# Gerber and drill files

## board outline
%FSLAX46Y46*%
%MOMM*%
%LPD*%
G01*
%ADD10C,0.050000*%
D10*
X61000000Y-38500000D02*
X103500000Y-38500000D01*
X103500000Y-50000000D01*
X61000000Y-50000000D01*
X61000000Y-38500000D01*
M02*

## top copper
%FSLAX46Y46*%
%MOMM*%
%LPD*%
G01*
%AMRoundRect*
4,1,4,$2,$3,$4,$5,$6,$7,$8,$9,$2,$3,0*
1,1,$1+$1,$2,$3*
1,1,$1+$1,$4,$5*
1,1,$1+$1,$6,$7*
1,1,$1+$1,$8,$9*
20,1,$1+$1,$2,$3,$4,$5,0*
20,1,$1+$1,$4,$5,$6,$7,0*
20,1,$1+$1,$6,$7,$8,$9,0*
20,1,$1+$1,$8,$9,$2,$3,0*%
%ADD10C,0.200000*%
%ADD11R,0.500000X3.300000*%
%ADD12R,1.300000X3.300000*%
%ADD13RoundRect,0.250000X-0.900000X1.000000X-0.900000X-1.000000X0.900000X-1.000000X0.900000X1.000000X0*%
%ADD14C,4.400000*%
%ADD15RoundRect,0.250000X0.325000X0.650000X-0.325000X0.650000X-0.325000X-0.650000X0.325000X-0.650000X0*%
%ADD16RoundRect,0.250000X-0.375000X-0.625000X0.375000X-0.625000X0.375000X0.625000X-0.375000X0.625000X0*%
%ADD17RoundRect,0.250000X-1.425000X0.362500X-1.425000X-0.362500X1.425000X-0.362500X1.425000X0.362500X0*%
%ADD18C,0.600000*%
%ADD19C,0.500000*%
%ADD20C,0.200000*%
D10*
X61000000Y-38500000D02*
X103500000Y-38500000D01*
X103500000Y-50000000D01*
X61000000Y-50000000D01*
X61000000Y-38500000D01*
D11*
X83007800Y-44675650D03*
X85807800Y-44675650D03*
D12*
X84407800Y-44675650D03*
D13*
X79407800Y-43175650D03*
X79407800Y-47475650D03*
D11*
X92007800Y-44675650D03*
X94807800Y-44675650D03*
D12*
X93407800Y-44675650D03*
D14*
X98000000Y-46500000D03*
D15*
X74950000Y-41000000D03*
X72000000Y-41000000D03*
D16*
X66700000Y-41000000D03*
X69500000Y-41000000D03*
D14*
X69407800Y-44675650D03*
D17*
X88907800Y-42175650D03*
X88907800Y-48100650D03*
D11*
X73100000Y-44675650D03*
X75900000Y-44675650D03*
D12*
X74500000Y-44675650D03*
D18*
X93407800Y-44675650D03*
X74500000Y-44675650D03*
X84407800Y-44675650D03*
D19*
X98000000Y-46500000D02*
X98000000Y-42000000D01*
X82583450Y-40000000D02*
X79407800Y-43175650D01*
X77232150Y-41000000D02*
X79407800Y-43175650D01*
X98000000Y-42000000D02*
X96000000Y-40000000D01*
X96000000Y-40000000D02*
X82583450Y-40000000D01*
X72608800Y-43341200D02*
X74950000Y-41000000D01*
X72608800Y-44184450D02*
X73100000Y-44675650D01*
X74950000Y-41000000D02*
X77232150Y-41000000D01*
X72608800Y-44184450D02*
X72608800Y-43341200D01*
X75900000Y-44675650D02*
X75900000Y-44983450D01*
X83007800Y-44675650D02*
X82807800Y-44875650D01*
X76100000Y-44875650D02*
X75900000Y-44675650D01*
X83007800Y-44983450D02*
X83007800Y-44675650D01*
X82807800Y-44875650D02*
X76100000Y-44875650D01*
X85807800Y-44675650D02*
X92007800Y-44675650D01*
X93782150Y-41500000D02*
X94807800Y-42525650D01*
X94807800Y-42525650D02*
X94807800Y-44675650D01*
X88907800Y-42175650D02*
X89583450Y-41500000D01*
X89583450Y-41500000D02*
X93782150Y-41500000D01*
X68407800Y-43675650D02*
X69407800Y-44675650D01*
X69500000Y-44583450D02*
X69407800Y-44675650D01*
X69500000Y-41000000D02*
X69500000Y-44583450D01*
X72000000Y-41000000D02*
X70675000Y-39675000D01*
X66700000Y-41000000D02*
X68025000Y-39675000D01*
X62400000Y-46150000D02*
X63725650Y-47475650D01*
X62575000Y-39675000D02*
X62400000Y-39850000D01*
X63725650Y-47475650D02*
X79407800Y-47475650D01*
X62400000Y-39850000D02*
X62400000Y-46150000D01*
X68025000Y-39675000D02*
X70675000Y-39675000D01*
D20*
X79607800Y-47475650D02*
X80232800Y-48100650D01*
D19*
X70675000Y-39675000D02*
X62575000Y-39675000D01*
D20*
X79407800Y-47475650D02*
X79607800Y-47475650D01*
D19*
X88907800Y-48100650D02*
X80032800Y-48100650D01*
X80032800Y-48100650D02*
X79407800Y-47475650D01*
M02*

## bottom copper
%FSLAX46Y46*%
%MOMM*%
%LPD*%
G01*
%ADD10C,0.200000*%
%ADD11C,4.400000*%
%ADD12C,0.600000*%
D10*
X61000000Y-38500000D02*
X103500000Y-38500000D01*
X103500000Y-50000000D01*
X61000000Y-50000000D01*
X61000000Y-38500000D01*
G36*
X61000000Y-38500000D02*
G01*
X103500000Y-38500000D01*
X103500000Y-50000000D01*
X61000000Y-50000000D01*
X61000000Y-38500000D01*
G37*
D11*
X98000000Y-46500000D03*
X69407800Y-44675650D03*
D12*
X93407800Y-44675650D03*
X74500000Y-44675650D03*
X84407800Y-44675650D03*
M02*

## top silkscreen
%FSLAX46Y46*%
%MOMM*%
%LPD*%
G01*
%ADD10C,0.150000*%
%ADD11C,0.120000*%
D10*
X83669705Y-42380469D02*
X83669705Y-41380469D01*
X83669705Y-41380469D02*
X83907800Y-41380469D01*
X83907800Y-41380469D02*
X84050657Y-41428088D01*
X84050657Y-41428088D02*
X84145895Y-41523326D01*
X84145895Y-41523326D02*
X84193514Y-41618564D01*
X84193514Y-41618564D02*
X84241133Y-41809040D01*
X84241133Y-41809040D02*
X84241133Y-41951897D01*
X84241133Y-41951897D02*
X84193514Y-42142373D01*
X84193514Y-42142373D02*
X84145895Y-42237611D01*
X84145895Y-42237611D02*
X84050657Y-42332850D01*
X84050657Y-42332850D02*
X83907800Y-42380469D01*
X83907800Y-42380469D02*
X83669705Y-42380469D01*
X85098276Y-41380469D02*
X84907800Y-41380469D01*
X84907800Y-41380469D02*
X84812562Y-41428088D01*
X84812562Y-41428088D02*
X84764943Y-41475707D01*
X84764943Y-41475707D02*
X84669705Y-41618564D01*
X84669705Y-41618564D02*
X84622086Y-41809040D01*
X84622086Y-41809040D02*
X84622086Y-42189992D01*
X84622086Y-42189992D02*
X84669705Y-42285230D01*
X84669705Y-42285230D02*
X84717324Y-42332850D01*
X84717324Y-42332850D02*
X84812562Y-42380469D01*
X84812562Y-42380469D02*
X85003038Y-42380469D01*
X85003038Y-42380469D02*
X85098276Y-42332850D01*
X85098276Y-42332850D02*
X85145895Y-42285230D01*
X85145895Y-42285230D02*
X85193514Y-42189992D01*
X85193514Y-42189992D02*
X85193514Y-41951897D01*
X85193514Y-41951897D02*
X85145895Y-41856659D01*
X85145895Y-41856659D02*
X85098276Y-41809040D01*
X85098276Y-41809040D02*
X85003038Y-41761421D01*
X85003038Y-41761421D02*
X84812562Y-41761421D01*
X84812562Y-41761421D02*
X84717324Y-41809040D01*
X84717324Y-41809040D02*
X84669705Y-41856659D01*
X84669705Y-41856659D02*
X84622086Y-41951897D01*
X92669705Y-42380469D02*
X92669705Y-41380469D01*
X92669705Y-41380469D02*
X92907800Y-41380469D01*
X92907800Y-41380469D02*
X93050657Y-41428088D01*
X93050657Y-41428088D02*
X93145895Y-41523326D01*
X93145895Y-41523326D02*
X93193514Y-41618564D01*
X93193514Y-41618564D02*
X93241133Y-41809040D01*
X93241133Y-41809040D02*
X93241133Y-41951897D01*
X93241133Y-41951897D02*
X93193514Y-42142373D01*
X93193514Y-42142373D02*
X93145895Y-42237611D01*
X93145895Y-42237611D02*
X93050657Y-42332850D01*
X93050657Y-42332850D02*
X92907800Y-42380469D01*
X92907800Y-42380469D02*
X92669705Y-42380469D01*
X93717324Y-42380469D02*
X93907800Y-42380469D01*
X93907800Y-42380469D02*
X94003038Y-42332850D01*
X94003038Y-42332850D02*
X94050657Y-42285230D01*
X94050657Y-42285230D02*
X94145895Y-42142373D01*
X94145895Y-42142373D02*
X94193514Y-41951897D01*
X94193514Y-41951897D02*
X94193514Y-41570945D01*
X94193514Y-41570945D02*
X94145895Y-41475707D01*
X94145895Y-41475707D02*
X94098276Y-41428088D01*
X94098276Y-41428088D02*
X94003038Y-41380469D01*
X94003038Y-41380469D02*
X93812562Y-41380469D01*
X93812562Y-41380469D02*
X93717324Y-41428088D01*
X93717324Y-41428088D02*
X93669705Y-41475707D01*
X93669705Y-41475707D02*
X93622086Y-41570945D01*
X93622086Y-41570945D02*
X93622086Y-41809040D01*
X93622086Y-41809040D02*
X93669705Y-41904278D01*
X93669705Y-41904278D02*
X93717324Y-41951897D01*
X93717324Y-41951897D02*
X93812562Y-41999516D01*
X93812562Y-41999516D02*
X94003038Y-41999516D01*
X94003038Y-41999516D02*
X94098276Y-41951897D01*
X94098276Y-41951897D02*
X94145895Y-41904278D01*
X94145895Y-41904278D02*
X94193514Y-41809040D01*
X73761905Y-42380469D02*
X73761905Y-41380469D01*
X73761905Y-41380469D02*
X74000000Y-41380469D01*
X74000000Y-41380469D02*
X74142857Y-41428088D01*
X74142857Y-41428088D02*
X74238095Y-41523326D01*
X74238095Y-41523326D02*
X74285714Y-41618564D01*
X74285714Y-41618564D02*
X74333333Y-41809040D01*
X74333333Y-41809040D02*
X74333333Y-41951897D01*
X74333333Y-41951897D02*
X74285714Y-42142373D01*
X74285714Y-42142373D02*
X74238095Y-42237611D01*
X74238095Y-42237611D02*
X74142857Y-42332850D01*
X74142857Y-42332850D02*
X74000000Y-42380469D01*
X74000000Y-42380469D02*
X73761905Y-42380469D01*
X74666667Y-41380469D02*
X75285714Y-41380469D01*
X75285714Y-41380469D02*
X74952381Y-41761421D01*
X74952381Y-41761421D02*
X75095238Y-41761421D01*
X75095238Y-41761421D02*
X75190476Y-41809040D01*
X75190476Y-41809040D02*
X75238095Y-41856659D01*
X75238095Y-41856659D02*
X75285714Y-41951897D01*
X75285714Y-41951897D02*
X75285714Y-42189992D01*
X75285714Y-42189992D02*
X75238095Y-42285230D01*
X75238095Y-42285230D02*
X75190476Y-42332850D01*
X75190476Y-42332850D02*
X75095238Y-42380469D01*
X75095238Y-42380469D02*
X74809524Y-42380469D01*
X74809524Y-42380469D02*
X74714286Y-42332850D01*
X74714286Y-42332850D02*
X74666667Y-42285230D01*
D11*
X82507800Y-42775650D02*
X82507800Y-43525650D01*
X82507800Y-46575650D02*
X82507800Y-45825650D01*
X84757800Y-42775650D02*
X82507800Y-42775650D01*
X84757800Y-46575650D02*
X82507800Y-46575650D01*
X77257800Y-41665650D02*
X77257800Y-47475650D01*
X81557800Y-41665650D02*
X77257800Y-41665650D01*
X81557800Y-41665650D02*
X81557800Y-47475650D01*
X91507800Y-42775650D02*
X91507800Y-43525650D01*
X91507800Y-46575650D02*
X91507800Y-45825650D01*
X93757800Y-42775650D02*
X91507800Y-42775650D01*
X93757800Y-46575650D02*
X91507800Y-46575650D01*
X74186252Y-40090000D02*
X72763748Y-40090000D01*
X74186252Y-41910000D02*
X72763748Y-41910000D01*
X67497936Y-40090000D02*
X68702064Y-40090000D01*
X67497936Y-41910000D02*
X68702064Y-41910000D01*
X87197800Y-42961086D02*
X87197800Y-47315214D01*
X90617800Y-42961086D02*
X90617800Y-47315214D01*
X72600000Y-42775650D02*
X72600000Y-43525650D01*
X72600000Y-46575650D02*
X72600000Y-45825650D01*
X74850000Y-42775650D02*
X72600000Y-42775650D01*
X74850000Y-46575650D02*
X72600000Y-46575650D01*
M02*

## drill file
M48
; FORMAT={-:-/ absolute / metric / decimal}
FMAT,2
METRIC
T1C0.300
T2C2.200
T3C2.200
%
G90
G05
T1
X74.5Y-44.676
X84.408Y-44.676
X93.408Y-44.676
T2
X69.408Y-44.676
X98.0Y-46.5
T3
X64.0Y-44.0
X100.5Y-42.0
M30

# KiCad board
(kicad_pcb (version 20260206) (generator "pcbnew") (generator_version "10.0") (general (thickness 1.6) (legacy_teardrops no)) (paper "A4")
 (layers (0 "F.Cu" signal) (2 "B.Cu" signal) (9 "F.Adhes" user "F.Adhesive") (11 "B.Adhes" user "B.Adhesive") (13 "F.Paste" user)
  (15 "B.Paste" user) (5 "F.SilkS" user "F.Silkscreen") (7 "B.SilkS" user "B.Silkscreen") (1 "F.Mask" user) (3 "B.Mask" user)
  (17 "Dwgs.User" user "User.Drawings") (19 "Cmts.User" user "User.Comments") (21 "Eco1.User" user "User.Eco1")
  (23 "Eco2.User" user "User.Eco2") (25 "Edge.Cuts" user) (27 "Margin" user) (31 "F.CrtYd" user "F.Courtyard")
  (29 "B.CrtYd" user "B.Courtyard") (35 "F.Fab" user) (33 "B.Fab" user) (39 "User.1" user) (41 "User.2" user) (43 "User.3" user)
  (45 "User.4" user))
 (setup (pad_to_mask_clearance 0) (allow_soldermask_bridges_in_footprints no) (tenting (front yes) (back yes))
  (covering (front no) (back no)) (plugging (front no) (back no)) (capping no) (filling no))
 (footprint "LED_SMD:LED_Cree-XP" (layer "F.Cu") (at 84.4078 44.67565)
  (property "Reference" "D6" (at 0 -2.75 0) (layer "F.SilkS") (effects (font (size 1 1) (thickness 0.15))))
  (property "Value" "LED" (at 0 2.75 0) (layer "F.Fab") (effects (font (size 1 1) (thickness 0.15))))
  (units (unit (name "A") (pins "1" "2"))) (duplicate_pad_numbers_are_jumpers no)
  (fp_line (start -1.9 -1.9) (end -1.9 -1.15) (stroke (width 0.12) (type solid)) (layer "F.SilkS"))
  (fp_line (start -1.9 1.9) (end -1.9 1.15) (stroke (width 0.12) (type solid)) (layer "F.SilkS"))
  (fp_line (start 0.35 -1.9) (end -1.9 -1.9) (stroke (width 0.12) (type solid)) (layer "F.SilkS"))
  (fp_line (start 0.35 1.9) (end -1.9 1.9) (stroke (width 0.12) (type solid)) (layer "F.SilkS"))
  (pad "" smd rect (at 0 -1) (size 1.01 0.75) (layers "F.Paste"))
  (pad "" smd rect (at 0 0) (size 1.01 0.75) (layers "F.Paste"))
  (pad "" smd rect (at 0 1) (size 1.01 0.75) (layers "F.Paste"))
  (pad "1" smd rect (at -1.4 0) (size 0.5 3.3) (layers "F.Cu" "F.Mask" "F.Paste") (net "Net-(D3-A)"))
  (pad "2" smd rect (at 1.4 0) (size 0.5 3.3) (layers "F.Cu" "F.Mask" "F.Paste") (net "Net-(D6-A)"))
  (pad "3" smd rect (at 0 0) (size 1.3 3.3) (layers "F.Cu" "F.Mask") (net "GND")))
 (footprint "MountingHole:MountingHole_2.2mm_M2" (layer "F.Cu") (at 64 44)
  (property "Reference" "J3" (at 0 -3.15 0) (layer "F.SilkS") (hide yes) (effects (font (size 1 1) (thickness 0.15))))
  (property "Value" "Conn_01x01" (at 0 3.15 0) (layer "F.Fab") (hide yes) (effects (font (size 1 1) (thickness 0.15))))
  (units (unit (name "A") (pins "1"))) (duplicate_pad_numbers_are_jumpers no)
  (pad "" np_thru_hole circle (at 0 0) (size 2.2 2.2) (drill 2.2) (layers "*.Cu" "*.Mask")))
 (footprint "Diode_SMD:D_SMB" (layer "F.Cu") (at 79.4078 45.32565 -90)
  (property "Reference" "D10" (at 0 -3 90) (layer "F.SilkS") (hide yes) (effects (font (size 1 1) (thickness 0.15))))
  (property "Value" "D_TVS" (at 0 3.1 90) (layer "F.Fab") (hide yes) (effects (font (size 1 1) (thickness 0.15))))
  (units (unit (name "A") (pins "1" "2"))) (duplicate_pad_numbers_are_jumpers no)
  (fp_line (start -3.66 2.15) (end 2.15 2.15) (stroke (width 0.12) (type solid)) (layer "F.SilkS"))
  (fp_line (start -3.66 -2.15) (end -3.66 2.15) (stroke (width 0.12) (type solid)) (layer "F.SilkS"))
  (fp_line (start -3.66 -2.15) (end 2.15 -2.15) (stroke (width 0.12) (type solid)) (layer "F.SilkS"))
  (pad "1" smd roundrect (at -2.15 0 270) (size 2.5 2.3) (layers "F.Cu" "F.Mask" "F.Paste") (roundrect_rratio 0.1086956522) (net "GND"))
  (pad "2" smd roundrect (at 2.15 0 270) (size 2.5 2.3) (layers "F.Cu" "F.Mask" "F.Paste") (roundrect_rratio 0.1086956522)
   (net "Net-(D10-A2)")))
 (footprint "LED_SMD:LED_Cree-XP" (layer "F.Cu") (at 93.4078 44.67565)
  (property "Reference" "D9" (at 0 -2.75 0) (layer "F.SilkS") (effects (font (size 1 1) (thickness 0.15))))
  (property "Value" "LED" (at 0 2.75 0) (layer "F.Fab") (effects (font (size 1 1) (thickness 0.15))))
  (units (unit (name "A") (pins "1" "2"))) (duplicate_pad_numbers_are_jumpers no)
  (fp_line (start -1.9 -1.9) (end -1.9 -1.15) (stroke (width 0.12) (type solid)) (layer "F.SilkS"))
  (fp_line (start -1.9 1.9) (end -1.9 1.15) (stroke (width 0.12) (type solid)) (layer "F.SilkS"))
  (fp_line (start 0.35 -1.9) (end -1.9 -1.9) (stroke (width 0.12) (type solid)) (layer "F.SilkS"))
  (fp_line (start 0.35 1.9) (end -1.9 1.9) (stroke (width 0.12) (type solid)) (layer "F.SilkS"))
  (pad "" smd rect (at 0 -1) (size 1.01 0.75) (layers "F.Paste"))
  (pad "" smd rect (at 0 0) (size 1.01 0.75) (layers "F.Paste"))
  (pad "" smd rect (at 0 1) (size 1.01 0.75) (layers "F.Paste"))
  (pad "1" smd rect (at -1.4 0) (size 0.5 3.3) (layers "F.Cu" "F.Mask" "F.Paste") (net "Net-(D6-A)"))
  (pad "2" smd rect (at 1.4 0) (size 0.5 3.3) (layers "F.Cu" "F.Mask" "F.Paste") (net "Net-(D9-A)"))
  (pad "3" smd rect (at 0 0) (size 1.3 3.3) (layers "F.Cu" "F.Mask") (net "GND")))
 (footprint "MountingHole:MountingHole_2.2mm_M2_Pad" (layer "F.Cu") (at 98 46.5)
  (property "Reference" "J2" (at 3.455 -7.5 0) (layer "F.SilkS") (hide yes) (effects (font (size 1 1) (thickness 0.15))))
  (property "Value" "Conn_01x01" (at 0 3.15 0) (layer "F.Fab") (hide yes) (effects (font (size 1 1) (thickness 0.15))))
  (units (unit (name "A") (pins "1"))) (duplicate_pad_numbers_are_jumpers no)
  (pad "1" thru_hole circle (at 0 0) (size 4.4 4.4) (drill 2.2) (layers "*.Cu" "*.Mask") (remove_unused_layers no) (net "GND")
   (zone_connect 2)))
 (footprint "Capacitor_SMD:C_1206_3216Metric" (layer "F.Cu") (at 73.475 41 180)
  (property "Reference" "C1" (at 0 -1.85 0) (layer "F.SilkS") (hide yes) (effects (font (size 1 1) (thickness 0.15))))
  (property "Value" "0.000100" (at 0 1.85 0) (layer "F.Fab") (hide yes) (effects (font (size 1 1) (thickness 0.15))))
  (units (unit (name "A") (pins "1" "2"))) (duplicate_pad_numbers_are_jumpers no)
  (fp_line (start -0.711252 0.91) (end 0.711252 0.91) (stroke (width 0.12) (type solid)) (layer "F.SilkS"))
  (fp_line (start -0.711252 -0.91) (end 0.711252 -0.91) (stroke (width 0.12) (type solid)) (layer "F.SilkS"))
  (pad "1" smd roundrect (at -1.475 0 180) (size 1.15 1.8) (layers "F.Cu" "F.Mask" "F.Paste") (roundrect_rratio 0.217391) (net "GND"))
  (pad "2" smd roundrect (at 1.475 0 180) (size 1.15 1.8) (layers "F.Cu" "F.Mask" "F.Paste") (roundrect_rratio 0.217391)
   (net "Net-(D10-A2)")))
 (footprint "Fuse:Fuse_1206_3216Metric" (layer "F.Cu") (at 68.1 41)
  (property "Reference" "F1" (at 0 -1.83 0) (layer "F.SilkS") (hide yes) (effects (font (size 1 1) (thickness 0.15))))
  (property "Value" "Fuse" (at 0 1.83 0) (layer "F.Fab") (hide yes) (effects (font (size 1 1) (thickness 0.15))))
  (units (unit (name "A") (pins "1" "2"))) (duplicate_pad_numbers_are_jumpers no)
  (fp_line (start -0.602064 -0.91) (end 0.602064 -0.91) (stroke (width 0.12) (type solid)) (layer "F.SilkS"))
  (fp_line (start -0.602064 0.91) (end 0.602064 0.91) (stroke (width 0.12) (type solid)) (layer "F.SilkS"))
  (pad "1" smd roundrect (at -1.4 0) (size 1.25 1.75) (layers "F.Cu" "F.Mask" "F.Paste") (roundrect_rratio 0.2) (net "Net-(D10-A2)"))
  (pad "2" smd roundrect (at 1.4 0) (size 1.25 1.75) (layers "F.Cu" "F.Mask" "F.Paste") (roundrect_rratio 0.2) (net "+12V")))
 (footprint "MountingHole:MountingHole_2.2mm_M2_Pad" (layer "F.Cu") (at 69.4078 44.67565)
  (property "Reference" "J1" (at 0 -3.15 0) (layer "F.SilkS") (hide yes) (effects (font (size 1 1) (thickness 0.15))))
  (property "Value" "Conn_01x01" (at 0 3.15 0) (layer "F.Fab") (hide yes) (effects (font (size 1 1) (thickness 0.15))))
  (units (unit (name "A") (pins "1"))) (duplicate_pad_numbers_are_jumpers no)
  (pad "1" thru_hole circle (at 0 0) (size 4.4 4.4) (drill 2.2) (layers "*.Cu" "*.Mask") (remove_unused_layers no) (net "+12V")
   (zone_connect 2)))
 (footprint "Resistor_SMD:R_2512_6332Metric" (layer "F.Cu") (at 88.9078 45.13815 -90)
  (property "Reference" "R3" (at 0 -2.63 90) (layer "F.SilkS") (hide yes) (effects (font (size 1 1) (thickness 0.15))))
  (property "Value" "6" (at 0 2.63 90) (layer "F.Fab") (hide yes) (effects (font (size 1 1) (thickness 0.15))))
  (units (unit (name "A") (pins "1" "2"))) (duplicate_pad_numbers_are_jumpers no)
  (fp_line (start -2.177064 1.71) (end 2.177064 1.71) (stroke (width 0.12) (type solid)) (layer "F.SilkS"))
  (fp_line (start -2.177064 -1.71) (end 2.177064 -1.71) (stroke (width 0.12) (type solid)) (layer "F.SilkS"))
  (pad "1" smd roundrect (at -2.9625 0 270) (size 1.225 3.35) (layers "F.Cu" "F.Mask" "F.Paste") (roundrect_rratio 0.204082)
   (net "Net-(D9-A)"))
  (pad "2" smd roundrect (at 2.9625 0 270) (size 1.225 3.35) (layers "F.Cu" "F.Mask" "F.Paste") (roundrect_rratio 0.204082)
   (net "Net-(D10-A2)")))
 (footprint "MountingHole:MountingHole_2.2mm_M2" (layer "F.Cu") (at 100.5 42)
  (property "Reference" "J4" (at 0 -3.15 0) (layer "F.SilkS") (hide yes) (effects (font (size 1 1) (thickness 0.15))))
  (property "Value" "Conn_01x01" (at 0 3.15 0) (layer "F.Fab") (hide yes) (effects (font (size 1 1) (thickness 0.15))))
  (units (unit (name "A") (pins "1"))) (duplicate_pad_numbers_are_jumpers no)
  (pad "" np_thru_hole circle (at 0 0) (size 2.2 2.2) (drill 2.2) (layers "*.Cu" "*.Mask")))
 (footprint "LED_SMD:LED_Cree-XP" (layer "F.Cu") (at 74.5 44.67565)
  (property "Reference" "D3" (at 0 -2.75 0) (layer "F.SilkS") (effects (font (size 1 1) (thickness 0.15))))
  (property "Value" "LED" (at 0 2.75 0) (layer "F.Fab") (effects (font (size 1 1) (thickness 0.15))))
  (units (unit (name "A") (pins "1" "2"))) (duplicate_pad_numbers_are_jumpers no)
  (fp_line (start -1.9 -1.9) (end -1.9 -1.15) (stroke (width 0.12) (type solid)) (layer "F.SilkS"))
  (fp_line (start -1.9 1.9) (end -1.9 1.15) (stroke (width 0.12) (type solid)) (layer "F.SilkS"))
  (fp_line (start 0.35 -1.9) (end -1.9 -1.9) (stroke (width 0.12) (type solid)) (layer "F.SilkS"))
  (fp_line (start 0.35 1.9) (end -1.9 1.9) (stroke (width 0.12) (type solid)) (layer "F.SilkS"))
  (pad "" smd rect (at 0 -1) (size 1.01 0.75) (layers "F.Paste"))
  (pad "" smd rect (at 0 0) (size 1.01 0.75) (layers "F.Paste"))
  (pad "" smd rect (at 0 1) (size 1.01 0.75) (layers "F.Paste"))
  (pad "1" smd rect (at -1.4 0) (size 0.5 3.3) (layers "F.Cu" "F.Mask" "F.Paste") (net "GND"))
  (pad "2" smd rect (at 1.4 0) (size 0.5 3.3) (layers "F.Cu" "F.Mask" "F.Paste") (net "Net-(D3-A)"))
  (pad "3" smd rect (at 0 0) (size 1.3 3.3) (layers "F.Cu" "F.Mask") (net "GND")))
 (gr_rect (start 61 38.5) (end 103.5 50) (stroke (width 0.2) (type default)) (fill no) (layer "F.Cu"))
 (gr_rect (start 61 38.5) (end 103.5 50) (stroke (width 0.2) (type solid)) (fill yes) (layer "B.Cu") (net "GND"))
 (gr_rect (start 61 38.5) (end 103.5 50) (stroke (width 0.05) (type default)) (fill no) (layer "Edge.Cuts"))
 (segment (start 98 46.5) (end 98 42) (width 0.5) (layer "F.Cu") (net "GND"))
 (segment (start 82.58345 40) (end 79.4078 43.17565) (width 0.5) (layer "F.Cu") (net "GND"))
 (segment (start 77.23215 41) (end 79.4078 43.17565) (width 0.5) (layer "F.Cu") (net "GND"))
 (segment (start 98 42) (end 96 40) (width 0.5) (layer "F.Cu") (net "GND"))
 (segment (start 96 40) (end 82.58345 40) (width 0.5) (layer "F.Cu") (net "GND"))
 (segment (start 72.6088 43.3412) (end 74.95 41) (width 0.5) (layer "F.Cu") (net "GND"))
 (segment (start 72.6088 44.18445) (end 73.1 44.67565) (width 0.5) (layer "F.Cu") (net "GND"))
 (segment (start 74.95 41) (end 77.23215 41) (width 0.5) (layer "F.Cu") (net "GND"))
 (segment (start 72.6088 44.18445) (end 72.6088 43.3412) (width 0.5) (layer "F.Cu") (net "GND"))
 (via (at 93.4078 44.67565) (size 0.6) (drill 0.3) (layers "F.Cu" "B.Cu") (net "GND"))
 (via (at 74.5 44.67565) (size 0.6) (drill 0.3) (layers "F.Cu" "B.Cu") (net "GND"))
 (via (at 84.4078 44.67565) (size 0.6) (drill 0.3) (layers "F.Cu" "B.Cu") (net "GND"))
 (segment (start 75.9 44.67565) (end 75.9 44.98345) (width 0.5) (layer "F.Cu") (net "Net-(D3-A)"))
 (segment (start 83.0078 44.67565) (end 82.8078 44.87565) (width 0.5) (layer "F.Cu") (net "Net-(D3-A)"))
 (segment (start 76.1 44.87565) (end 75.9 44.67565) (width 0.5) (layer "F.Cu") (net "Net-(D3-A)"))
 (segment (start 83.0078 44.98345) (end 83.0078 44.67565) (width 0.5) (layer "F.Cu") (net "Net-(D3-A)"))
 (segment (start 82.8078 44.87565) (end 76.1 44.87565) (width 0.5) (layer "F.Cu") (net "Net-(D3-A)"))
 (segment (start 85.8078 44.67565) (end 92.0078 44.67565) (width 0.5) (layer "F.Cu") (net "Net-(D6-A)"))
 (segment (start 93.78215 41.5) (end 94.8078 42.52565) (width 0.5) (layer "F.Cu") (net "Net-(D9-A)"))
 (segment (start 94.8078 42.52565) (end 94.8078 44.67565) (width 0.5) (layer "F.Cu") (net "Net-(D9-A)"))
 (segment (start 88.9078 42.17565) (end 89.58345 41.5) (width 0.5) (layer "F.Cu") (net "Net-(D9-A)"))
 (segment (start 89.58345 41.5) (end 93.78215 41.5) (width 0.5) (layer "F.Cu") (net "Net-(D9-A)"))
 (segment (start 68.4078 43.67565) (end 69.4078 44.67565) (width 0.5) (layer "F.Cu") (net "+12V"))
 (segment (start 69.5 44.58345) (end 69.4078 44.67565) (width 0.5) (layer "F.Cu") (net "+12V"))
 (segment (start 69.5 41) (end 69.5 44.58345) (width 0.5) (layer "F.Cu") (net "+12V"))
 (segment (start 72 41) (end 70.675 39.675) (width 0.5) (layer "F.Cu") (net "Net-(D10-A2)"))
 (segment (start 66.7 41) (end 68.025 39.675) (width 0.5) (layer "F.Cu") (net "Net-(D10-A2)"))
 (segment (start 62.4 46.15) (end 63.72565 47.47565) (width 0.5) (layer "F.Cu") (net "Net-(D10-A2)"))
 (segment (start 62.575 39.675) (end 62.4 39.85) (width 0.5) (layer "F.Cu") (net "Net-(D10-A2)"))
 (segment (start 63.72565 47.47565) (end 79.4078 47.47565) (width 0.5) (layer "F.Cu") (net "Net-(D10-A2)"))
 (segment (start 62.4 39.85) (end 62.4 46.15) (width 0.5) (layer "F.Cu") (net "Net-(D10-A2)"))
 (segment (start 68.025 39.675) (end 70.675 39.675) (width 0.5) (layer "F.Cu") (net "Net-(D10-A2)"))
 (segment (start 79.6078 47.47565) (end 80.2328 48.10065) (width 0.2) (layer "F.Cu") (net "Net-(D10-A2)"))
 (segment (start 70.675 39.675) (end 62.575 39.675) (width 0.5) (layer "F.Cu") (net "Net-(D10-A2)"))
 (segment (start 79.4078 47.47565) (end 79.6078 47.47565) (width 0.2) (layer "F.Cu") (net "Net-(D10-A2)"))
 (segment (start 88.9078 48.10065) (end 80.0328 48.10065) (width 0.5) (layer "F.Cu") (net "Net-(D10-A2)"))
 (segment (start 80.0328 48.10065) (end 79.4078 47.47565) (width 0.5) (layer "F.Cu") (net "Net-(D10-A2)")))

